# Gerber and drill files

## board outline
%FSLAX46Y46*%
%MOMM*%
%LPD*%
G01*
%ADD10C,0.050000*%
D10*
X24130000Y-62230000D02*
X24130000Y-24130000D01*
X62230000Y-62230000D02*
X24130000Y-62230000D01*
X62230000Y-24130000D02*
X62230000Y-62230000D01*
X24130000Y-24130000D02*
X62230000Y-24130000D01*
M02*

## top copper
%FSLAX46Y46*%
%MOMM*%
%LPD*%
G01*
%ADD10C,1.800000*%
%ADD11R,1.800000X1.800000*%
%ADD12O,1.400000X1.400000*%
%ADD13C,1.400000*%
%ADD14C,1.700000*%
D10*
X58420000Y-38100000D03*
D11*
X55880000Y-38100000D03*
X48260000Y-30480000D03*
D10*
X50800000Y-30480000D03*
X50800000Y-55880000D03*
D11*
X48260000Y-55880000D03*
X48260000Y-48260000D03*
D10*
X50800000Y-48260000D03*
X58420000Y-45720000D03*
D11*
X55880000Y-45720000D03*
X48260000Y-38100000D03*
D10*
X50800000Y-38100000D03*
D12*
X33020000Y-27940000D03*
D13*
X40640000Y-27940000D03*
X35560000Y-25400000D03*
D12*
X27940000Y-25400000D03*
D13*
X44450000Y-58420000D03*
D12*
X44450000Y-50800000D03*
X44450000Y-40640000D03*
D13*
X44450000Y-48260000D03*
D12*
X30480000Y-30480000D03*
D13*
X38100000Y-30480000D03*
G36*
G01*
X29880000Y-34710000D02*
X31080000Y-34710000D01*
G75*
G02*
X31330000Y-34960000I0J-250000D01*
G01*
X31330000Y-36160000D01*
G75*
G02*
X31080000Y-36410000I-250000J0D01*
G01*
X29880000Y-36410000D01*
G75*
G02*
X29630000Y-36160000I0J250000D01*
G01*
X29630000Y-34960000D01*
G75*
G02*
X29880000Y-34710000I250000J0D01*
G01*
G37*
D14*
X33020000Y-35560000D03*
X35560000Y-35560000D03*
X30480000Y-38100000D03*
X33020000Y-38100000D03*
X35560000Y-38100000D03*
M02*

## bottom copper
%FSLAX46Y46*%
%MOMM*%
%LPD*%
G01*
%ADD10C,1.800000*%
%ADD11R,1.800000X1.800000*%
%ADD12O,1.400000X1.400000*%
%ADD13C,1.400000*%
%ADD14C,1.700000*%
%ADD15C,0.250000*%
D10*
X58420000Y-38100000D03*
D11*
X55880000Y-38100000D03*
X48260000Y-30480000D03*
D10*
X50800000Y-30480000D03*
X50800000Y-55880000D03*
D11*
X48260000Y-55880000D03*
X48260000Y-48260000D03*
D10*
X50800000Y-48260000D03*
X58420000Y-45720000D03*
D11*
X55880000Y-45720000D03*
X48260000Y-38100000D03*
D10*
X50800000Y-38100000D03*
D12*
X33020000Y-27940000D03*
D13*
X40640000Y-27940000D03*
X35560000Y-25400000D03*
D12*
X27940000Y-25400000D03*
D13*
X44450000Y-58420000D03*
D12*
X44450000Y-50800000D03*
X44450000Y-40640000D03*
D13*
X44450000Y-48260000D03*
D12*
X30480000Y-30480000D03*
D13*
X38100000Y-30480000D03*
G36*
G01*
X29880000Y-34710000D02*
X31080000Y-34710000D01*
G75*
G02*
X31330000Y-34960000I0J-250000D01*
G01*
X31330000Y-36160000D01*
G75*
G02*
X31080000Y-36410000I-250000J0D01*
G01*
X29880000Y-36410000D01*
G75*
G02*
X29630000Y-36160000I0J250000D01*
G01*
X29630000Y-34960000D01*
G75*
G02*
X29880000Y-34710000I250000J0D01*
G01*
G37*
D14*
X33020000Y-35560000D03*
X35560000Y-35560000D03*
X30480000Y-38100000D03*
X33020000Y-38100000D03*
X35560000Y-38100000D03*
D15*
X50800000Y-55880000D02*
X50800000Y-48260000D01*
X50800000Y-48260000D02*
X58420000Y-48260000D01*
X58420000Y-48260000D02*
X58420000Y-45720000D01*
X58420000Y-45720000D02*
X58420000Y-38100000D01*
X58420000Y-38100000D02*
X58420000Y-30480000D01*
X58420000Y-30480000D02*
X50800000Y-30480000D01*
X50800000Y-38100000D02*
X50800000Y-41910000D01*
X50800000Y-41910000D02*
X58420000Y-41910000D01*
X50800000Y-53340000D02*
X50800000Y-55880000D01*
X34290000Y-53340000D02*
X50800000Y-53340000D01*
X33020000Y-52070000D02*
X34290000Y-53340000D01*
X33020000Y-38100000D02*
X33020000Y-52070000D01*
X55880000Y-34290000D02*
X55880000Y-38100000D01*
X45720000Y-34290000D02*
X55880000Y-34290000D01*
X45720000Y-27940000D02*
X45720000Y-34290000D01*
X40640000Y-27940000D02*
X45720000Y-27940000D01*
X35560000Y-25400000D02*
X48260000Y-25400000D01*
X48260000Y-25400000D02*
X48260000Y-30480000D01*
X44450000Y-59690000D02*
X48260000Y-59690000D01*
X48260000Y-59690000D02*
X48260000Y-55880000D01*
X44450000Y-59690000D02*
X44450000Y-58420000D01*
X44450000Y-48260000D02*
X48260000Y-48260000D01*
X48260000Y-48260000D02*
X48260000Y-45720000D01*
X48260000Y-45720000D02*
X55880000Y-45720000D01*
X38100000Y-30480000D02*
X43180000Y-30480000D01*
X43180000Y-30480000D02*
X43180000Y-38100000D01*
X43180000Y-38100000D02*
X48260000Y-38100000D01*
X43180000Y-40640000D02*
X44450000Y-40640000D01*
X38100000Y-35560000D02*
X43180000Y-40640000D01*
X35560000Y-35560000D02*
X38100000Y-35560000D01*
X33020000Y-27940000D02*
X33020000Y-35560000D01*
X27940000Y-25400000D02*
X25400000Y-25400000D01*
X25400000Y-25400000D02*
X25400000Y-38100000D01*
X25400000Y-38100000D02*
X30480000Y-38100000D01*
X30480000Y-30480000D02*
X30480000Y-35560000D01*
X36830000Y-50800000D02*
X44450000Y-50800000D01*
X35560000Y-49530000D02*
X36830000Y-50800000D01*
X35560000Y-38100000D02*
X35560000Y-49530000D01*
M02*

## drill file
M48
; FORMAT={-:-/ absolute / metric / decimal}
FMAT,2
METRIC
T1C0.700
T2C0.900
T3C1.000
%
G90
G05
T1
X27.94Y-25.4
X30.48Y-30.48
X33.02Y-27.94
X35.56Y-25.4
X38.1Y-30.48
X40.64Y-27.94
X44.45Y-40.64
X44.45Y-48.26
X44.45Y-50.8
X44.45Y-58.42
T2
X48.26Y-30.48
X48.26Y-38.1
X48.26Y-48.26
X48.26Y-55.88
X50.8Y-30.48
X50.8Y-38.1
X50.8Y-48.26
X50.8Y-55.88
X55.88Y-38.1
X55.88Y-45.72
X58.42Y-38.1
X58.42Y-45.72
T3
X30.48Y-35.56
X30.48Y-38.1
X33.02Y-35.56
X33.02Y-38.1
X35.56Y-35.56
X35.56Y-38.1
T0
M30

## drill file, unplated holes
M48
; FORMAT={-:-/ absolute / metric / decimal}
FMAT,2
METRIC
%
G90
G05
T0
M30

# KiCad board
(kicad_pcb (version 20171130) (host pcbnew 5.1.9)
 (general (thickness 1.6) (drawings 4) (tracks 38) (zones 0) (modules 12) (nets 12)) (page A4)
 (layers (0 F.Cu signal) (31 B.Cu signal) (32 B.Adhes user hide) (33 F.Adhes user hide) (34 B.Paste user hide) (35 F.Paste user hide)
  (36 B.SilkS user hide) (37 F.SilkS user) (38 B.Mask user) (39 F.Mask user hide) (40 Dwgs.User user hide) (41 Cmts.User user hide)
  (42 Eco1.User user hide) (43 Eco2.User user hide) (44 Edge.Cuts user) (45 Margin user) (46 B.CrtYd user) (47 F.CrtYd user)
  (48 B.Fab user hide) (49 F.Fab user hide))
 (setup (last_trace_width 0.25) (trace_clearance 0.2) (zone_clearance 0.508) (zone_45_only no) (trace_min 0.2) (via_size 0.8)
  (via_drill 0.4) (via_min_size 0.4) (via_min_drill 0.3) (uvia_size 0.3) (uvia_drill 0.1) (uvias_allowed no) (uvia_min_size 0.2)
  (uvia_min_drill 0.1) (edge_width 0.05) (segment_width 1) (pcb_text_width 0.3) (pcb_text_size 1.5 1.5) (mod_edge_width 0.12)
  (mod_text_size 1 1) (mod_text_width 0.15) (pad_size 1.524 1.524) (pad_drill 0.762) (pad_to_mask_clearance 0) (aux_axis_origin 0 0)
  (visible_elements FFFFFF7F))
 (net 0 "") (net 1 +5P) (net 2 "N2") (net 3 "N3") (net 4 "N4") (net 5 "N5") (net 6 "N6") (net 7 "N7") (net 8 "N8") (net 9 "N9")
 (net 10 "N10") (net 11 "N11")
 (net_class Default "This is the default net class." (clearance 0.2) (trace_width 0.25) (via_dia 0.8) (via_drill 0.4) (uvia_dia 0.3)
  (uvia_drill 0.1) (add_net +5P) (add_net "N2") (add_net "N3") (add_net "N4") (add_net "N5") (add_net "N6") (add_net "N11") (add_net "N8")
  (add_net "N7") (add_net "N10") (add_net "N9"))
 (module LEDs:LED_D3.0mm (layer F.Cu) (at 55.88 38.1)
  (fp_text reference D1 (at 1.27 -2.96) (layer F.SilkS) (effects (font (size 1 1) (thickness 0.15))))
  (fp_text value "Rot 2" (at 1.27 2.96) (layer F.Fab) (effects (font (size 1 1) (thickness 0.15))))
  (pad 2 thru_hole circle (at 2.54 0) (size 1.8 1.8) (drill 0.9) (layers *.Cu *.Mask) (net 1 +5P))
  (pad 1 thru_hole rect (at 0 0) (size 1.8 1.8) (drill 0.9) (layers *.Cu *.Mask) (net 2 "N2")))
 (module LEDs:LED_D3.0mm (layer F.Cu) (at 48.26 30.48)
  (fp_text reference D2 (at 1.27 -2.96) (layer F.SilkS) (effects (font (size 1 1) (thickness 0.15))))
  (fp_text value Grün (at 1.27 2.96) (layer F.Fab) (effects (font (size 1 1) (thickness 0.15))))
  (pad 1 thru_hole rect (at 0 0) (size 1.8 1.8) (drill 0.9) (layers *.Cu *.Mask) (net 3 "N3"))
  (pad 2 thru_hole circle (at 2.54 0) (size 1.8 1.8) (drill 0.9) (layers *.Cu *.Mask) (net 1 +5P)))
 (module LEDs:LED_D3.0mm (layer F.Cu) (at 48.26 55.88)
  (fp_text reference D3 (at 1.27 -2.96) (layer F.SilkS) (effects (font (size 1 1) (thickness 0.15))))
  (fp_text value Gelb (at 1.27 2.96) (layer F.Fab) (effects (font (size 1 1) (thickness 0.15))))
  (pad 2 thru_hole circle (at 2.54 0) (size 1.8 1.8) (drill 0.9) (layers *.Cu *.Mask) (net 1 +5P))
  (pad 1 thru_hole rect (at 0 0) (size 1.8 1.8) (drill 0.9) (layers *.Cu *.Mask) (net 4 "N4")))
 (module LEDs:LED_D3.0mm (layer F.Cu) (at 48.26 48.26)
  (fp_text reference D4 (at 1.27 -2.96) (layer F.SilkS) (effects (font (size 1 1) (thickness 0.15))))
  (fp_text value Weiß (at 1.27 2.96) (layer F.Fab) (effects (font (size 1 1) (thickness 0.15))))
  (pad 1 thru_hole rect (at 0 0) (size 1.8 1.8) (drill 0.9) (layers *.Cu *.Mask) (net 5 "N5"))
  (pad 2 thru_hole circle (at 2.54 0) (size 1.8 1.8) (drill 0.9) (layers *.Cu *.Mask) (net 1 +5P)))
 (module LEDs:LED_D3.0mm (layer F.Cu) (at 55.88 45.72)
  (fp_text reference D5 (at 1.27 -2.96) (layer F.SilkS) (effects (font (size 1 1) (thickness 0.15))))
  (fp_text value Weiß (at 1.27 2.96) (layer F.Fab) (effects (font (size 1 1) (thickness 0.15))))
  (pad 2 thru_hole circle (at 2.54 0) (size 1.8 1.8) (drill 0.9) (layers *.Cu *.Mask) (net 1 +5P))
  (pad 1 thru_hole rect (at 0 0) (size 1.8 1.8) (drill 0.9) (layers *.Cu *.Mask) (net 5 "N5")))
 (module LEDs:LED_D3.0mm (layer F.Cu) (at 48.26 38.1)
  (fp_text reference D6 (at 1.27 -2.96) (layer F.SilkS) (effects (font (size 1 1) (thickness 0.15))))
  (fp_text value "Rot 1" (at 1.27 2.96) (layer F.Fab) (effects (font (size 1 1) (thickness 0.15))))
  (pad 1 thru_hole rect (at 0 0) (size 1.8 1.8) (drill 0.9) (layers *.Cu *.Mask) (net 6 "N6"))
  (pad 2 thru_hole circle (at 2.54 0) (size 1.8 1.8) (drill 0.9) (layers *.Cu *.Mask) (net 1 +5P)))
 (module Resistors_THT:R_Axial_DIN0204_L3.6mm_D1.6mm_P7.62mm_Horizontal (layer F.Cu) (at 40.64 27.94 180)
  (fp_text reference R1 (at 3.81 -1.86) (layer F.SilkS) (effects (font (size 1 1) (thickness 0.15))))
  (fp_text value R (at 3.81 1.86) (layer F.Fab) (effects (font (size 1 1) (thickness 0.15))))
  (pad 2 thru_hole oval (at 7.62 0 180) (size 1.4 1.4) (drill 0.7) (layers *.Cu *.Mask) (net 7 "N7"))
  (pad 1 thru_hole circle (at 0 0 180) (size 1.4 1.4) (drill 0.7) (layers *.Cu *.Mask) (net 2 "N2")))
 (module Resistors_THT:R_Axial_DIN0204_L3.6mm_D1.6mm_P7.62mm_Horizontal (layer F.Cu) (at 35.56 25.4 180)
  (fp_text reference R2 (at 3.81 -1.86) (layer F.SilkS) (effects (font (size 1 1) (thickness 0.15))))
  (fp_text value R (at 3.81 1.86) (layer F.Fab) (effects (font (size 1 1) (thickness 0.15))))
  (pad 1 thru_hole circle (at 0 0 180) (size 1.4 1.4) (drill 0.7) (layers *.Cu *.Mask) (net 3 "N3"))
  (pad 2 thru_hole oval (at 7.62 0 180) (size 1.4 1.4) (drill 0.7) (layers *.Cu *.Mask) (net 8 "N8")))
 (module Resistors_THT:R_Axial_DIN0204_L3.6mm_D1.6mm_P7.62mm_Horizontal (layer F.Cu) (at 44.45 58.42 90)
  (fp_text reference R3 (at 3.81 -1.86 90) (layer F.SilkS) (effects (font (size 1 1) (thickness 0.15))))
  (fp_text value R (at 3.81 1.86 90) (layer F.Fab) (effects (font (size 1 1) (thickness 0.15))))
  (pad 1 thru_hole circle (at 0 0 90) (size 1.4 1.4) (drill 0.7) (layers *.Cu *.Mask) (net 4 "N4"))
  (pad 2 thru_hole oval (at 7.62 0 90) (size 1.4 1.4) (drill 0.7) (layers *.Cu *.Mask) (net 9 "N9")))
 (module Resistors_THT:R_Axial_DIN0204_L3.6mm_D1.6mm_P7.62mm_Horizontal (layer F.Cu) (at 44.45 48.26 90)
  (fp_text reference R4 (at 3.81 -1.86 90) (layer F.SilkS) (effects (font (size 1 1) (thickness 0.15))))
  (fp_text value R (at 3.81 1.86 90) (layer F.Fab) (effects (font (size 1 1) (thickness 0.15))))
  (pad 2 thru_hole oval (at 7.62 0 90) (size 1.4 1.4) (drill 0.7) (layers *.Cu *.Mask) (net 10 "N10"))
  (pad 1 thru_hole circle (at 0 0 90) (size 1.4 1.4) (drill 0.7) (layers *.Cu *.Mask) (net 5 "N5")))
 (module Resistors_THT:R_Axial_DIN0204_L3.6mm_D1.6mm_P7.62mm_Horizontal (layer F.Cu) (at 38.1 30.48 180)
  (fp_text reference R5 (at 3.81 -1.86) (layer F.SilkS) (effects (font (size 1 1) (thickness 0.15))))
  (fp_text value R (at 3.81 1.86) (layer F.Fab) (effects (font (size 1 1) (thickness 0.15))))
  (pad 2 thru_hole oval (at 7.62 0 180) (size 1.4 1.4) (drill 0.7) (layers *.Cu *.Mask) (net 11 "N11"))
  (pad 1 thru_hole circle (at 0 0 180) (size 1.4 1.4) (drill 0.7) (layers *.Cu *.Mask) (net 6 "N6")))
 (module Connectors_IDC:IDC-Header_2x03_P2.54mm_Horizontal (layer B.Cu) (at 30.48 35.56 270)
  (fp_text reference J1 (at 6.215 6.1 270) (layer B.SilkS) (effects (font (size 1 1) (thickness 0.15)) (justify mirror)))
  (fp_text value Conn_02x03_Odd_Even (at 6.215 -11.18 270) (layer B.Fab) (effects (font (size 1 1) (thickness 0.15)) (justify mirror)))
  (pad 1 thru_hole roundrect (at 0 0 270) (size 1.7 1.7) (drill 1) (layers *.Cu *.Mask) (roundrect_rratio 0.1470588235294118) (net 11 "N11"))
  (pad 3 thru_hole circle (at 0 -2.54 270) (size 1.7 1.7) (drill 1) (layers *.Cu *.Mask) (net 7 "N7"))
  (pad 5 thru_hole circle (at 0 -5.08 270) (size 1.7 1.7) (drill 1) (layers *.Cu *.Mask) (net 10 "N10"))
  (pad 2 thru_hole circle (at 2.54 0 270) (size 1.7 1.7) (drill 1) (layers *.Cu *.Mask) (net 8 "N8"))
  (pad 4 thru_hole circle (at 2.54 -2.54 270) (size 1.7 1.7) (drill 1) (layers *.Cu *.Mask) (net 1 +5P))
  (pad 6 thru_hole circle (at 2.54 -5.08 270) (size 1.7 1.7) (drill 1) (layers *.Cu *.Mask) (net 9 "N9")))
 (gr_line (start 24.13 62.23) (end 24.13 24.13) (layer Edge.Cuts) (width 0.05))
 (gr_line (start 62.23 62.23) (end 24.13 62.23) (layer Edge.Cuts) (width 0.05))
 (gr_line (start 62.23 24.13) (end 62.23 62.23) (layer Edge.Cuts) (width 0.05))
 (gr_line (start 24.13 24.13) (end 62.23 24.13) (layer Edge.Cuts) (width 0.05))
 (segment (start 50.8 55.88) (end 50.8 48.26) (width 0.25) (layer B.Cu) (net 1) (status 30))
 (segment (start 50.8 48.26) (end 58.42 48.26) (width 0.25) (layer B.Cu) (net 1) (status 10))
 (segment (start 58.42 48.26) (end 58.42 45.72) (width 0.25) (layer B.Cu) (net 1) (status 20))
 (segment (start 58.42 45.72) (end 58.42 38.1) (width 0.25) (layer B.Cu) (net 1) (status 30))
 (segment (start 58.42 38.1) (end 58.42 30.48) (width 0.25) (layer B.Cu) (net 1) (status 10))
 (segment (start 58.42 30.48) (end 50.8 30.48) (width 0.25) (layer B.Cu) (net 1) (status 20))
 (segment (start 50.8 38.1) (end 50.8 41.91) (width 0.25) (layer B.Cu) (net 1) (status 10))
 (segment (start 50.8 41.91) (end 58.42 41.91) (width 0.25) (layer B.Cu) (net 1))
 (segment (start 50.8 53.34) (end 50.8 55.88) (width 0.25) (layer B.Cu) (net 1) (status 20))
 (segment (start 34.29 53.34) (end 50.8 53.34) (width 0.25) (layer B.Cu) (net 1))
 (segment (start 33.02 52.07) (end 34.29 53.34) (width 0.25) (layer B.Cu) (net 1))
 (segment (start 33.02 38.1) (end 33.02 52.07) (width 0.25) (layer B.Cu) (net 1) (status 10))
 (segment (start 55.88 34.29) (end 55.88 38.1) (width 0.25) (layer B.Cu) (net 2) (status 20))
 (segment (start 45.72 34.29) (end 55.88 34.29) (width 0.25) (layer B.Cu) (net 2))
 (segment (start 45.72 27.94) (end 45.72 34.29) (width 0.25) (layer B.Cu) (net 2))
 (segment (start 40.64 27.94) (end 45.72 27.94) (width 0.25) (layer B.Cu) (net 2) (status 10))
 (segment (start 35.56 25.4) (end 48.26 25.4) (width 0.25) (layer B.Cu) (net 3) (status 10))
 (segment (start 48.26 25.4) (end 48.26 30.48) (width 0.25) (layer B.Cu) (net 3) (status 20))
 (segment (start 44.45 59.69) (end 48.26 59.69) (width 0.25) (layer B.Cu) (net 4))
 (segment (start 48.26 59.69) (end 48.26 55.88) (width 0.25) (layer B.Cu) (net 4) (status 20))
 (segment (start 44.45 59.69) (end 44.45 58.42) (width 0.25) (layer B.Cu) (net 4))
 (segment (start 44.45 48.26) (end 48.26 48.26) (width 0.25) (layer B.Cu) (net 5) (status 30))
 (segment (start 48.26 48.26) (end 48.26 45.72) (width 0.25) (layer B.Cu) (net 5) (status 10))
 (segment (start 48.26 45.72) (end 55.88 45.72) (width 0.25) (layer B.Cu) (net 5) (status 20))
 (segment (start 38.1 30.48) (end 43.18 30.48) (width 0.25) (layer B.Cu) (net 6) (status 10))
 (segment (start 43.18 30.48) (end 43.18 38.1) (width 0.25) (layer B.Cu) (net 6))
 (segment (start 43.18 38.1) (end 48.26 38.1) (width 0.25) (layer B.Cu) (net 6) (status 20))
 (segment (start 43.18 40.64) (end 44.45 40.64) (width 0.25) (layer B.Cu) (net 10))
 (segment (start 38.1 35.56) (end 43.18 40.64) (width 0.25) (layer B.Cu) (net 10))
 (segment (start 35.56 35.56) (end 38.1 35.56) (width 0.25) (layer B.Cu) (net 10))
 (segment (start 33.02 27.94) (end 33.02 35.56) (width 0.25) (layer B.Cu) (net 7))
 (segment (start 27.94 25.4) (end 25.4 25.4) (width 0.25) (layer B.Cu) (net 8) (status 10))
 (segment (start 25.4 25.4) (end 25.4 38.1) (width 0.25) (layer B.Cu) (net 8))
 (segment (start 25.4 38.1) (end 30.48 38.1) (width 0.25) (layer B.Cu) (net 8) (status 20))
 (segment (start 30.48 30.48) (end 30.48 35.56) (width 0.25) (layer B.Cu) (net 11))
 (segment (start 36.83 50.8) (end 44.45 50.8) (width 0.25) (layer B.Cu) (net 9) (status 20))
 (segment (start 35.56 49.53) (end 36.83 50.8) (width 0.25) (layer B.Cu) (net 9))
 (segment (start 35.56 38.1) (end 35.56 49.53) (width 0.25) (layer B.Cu) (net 9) (status 10)))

